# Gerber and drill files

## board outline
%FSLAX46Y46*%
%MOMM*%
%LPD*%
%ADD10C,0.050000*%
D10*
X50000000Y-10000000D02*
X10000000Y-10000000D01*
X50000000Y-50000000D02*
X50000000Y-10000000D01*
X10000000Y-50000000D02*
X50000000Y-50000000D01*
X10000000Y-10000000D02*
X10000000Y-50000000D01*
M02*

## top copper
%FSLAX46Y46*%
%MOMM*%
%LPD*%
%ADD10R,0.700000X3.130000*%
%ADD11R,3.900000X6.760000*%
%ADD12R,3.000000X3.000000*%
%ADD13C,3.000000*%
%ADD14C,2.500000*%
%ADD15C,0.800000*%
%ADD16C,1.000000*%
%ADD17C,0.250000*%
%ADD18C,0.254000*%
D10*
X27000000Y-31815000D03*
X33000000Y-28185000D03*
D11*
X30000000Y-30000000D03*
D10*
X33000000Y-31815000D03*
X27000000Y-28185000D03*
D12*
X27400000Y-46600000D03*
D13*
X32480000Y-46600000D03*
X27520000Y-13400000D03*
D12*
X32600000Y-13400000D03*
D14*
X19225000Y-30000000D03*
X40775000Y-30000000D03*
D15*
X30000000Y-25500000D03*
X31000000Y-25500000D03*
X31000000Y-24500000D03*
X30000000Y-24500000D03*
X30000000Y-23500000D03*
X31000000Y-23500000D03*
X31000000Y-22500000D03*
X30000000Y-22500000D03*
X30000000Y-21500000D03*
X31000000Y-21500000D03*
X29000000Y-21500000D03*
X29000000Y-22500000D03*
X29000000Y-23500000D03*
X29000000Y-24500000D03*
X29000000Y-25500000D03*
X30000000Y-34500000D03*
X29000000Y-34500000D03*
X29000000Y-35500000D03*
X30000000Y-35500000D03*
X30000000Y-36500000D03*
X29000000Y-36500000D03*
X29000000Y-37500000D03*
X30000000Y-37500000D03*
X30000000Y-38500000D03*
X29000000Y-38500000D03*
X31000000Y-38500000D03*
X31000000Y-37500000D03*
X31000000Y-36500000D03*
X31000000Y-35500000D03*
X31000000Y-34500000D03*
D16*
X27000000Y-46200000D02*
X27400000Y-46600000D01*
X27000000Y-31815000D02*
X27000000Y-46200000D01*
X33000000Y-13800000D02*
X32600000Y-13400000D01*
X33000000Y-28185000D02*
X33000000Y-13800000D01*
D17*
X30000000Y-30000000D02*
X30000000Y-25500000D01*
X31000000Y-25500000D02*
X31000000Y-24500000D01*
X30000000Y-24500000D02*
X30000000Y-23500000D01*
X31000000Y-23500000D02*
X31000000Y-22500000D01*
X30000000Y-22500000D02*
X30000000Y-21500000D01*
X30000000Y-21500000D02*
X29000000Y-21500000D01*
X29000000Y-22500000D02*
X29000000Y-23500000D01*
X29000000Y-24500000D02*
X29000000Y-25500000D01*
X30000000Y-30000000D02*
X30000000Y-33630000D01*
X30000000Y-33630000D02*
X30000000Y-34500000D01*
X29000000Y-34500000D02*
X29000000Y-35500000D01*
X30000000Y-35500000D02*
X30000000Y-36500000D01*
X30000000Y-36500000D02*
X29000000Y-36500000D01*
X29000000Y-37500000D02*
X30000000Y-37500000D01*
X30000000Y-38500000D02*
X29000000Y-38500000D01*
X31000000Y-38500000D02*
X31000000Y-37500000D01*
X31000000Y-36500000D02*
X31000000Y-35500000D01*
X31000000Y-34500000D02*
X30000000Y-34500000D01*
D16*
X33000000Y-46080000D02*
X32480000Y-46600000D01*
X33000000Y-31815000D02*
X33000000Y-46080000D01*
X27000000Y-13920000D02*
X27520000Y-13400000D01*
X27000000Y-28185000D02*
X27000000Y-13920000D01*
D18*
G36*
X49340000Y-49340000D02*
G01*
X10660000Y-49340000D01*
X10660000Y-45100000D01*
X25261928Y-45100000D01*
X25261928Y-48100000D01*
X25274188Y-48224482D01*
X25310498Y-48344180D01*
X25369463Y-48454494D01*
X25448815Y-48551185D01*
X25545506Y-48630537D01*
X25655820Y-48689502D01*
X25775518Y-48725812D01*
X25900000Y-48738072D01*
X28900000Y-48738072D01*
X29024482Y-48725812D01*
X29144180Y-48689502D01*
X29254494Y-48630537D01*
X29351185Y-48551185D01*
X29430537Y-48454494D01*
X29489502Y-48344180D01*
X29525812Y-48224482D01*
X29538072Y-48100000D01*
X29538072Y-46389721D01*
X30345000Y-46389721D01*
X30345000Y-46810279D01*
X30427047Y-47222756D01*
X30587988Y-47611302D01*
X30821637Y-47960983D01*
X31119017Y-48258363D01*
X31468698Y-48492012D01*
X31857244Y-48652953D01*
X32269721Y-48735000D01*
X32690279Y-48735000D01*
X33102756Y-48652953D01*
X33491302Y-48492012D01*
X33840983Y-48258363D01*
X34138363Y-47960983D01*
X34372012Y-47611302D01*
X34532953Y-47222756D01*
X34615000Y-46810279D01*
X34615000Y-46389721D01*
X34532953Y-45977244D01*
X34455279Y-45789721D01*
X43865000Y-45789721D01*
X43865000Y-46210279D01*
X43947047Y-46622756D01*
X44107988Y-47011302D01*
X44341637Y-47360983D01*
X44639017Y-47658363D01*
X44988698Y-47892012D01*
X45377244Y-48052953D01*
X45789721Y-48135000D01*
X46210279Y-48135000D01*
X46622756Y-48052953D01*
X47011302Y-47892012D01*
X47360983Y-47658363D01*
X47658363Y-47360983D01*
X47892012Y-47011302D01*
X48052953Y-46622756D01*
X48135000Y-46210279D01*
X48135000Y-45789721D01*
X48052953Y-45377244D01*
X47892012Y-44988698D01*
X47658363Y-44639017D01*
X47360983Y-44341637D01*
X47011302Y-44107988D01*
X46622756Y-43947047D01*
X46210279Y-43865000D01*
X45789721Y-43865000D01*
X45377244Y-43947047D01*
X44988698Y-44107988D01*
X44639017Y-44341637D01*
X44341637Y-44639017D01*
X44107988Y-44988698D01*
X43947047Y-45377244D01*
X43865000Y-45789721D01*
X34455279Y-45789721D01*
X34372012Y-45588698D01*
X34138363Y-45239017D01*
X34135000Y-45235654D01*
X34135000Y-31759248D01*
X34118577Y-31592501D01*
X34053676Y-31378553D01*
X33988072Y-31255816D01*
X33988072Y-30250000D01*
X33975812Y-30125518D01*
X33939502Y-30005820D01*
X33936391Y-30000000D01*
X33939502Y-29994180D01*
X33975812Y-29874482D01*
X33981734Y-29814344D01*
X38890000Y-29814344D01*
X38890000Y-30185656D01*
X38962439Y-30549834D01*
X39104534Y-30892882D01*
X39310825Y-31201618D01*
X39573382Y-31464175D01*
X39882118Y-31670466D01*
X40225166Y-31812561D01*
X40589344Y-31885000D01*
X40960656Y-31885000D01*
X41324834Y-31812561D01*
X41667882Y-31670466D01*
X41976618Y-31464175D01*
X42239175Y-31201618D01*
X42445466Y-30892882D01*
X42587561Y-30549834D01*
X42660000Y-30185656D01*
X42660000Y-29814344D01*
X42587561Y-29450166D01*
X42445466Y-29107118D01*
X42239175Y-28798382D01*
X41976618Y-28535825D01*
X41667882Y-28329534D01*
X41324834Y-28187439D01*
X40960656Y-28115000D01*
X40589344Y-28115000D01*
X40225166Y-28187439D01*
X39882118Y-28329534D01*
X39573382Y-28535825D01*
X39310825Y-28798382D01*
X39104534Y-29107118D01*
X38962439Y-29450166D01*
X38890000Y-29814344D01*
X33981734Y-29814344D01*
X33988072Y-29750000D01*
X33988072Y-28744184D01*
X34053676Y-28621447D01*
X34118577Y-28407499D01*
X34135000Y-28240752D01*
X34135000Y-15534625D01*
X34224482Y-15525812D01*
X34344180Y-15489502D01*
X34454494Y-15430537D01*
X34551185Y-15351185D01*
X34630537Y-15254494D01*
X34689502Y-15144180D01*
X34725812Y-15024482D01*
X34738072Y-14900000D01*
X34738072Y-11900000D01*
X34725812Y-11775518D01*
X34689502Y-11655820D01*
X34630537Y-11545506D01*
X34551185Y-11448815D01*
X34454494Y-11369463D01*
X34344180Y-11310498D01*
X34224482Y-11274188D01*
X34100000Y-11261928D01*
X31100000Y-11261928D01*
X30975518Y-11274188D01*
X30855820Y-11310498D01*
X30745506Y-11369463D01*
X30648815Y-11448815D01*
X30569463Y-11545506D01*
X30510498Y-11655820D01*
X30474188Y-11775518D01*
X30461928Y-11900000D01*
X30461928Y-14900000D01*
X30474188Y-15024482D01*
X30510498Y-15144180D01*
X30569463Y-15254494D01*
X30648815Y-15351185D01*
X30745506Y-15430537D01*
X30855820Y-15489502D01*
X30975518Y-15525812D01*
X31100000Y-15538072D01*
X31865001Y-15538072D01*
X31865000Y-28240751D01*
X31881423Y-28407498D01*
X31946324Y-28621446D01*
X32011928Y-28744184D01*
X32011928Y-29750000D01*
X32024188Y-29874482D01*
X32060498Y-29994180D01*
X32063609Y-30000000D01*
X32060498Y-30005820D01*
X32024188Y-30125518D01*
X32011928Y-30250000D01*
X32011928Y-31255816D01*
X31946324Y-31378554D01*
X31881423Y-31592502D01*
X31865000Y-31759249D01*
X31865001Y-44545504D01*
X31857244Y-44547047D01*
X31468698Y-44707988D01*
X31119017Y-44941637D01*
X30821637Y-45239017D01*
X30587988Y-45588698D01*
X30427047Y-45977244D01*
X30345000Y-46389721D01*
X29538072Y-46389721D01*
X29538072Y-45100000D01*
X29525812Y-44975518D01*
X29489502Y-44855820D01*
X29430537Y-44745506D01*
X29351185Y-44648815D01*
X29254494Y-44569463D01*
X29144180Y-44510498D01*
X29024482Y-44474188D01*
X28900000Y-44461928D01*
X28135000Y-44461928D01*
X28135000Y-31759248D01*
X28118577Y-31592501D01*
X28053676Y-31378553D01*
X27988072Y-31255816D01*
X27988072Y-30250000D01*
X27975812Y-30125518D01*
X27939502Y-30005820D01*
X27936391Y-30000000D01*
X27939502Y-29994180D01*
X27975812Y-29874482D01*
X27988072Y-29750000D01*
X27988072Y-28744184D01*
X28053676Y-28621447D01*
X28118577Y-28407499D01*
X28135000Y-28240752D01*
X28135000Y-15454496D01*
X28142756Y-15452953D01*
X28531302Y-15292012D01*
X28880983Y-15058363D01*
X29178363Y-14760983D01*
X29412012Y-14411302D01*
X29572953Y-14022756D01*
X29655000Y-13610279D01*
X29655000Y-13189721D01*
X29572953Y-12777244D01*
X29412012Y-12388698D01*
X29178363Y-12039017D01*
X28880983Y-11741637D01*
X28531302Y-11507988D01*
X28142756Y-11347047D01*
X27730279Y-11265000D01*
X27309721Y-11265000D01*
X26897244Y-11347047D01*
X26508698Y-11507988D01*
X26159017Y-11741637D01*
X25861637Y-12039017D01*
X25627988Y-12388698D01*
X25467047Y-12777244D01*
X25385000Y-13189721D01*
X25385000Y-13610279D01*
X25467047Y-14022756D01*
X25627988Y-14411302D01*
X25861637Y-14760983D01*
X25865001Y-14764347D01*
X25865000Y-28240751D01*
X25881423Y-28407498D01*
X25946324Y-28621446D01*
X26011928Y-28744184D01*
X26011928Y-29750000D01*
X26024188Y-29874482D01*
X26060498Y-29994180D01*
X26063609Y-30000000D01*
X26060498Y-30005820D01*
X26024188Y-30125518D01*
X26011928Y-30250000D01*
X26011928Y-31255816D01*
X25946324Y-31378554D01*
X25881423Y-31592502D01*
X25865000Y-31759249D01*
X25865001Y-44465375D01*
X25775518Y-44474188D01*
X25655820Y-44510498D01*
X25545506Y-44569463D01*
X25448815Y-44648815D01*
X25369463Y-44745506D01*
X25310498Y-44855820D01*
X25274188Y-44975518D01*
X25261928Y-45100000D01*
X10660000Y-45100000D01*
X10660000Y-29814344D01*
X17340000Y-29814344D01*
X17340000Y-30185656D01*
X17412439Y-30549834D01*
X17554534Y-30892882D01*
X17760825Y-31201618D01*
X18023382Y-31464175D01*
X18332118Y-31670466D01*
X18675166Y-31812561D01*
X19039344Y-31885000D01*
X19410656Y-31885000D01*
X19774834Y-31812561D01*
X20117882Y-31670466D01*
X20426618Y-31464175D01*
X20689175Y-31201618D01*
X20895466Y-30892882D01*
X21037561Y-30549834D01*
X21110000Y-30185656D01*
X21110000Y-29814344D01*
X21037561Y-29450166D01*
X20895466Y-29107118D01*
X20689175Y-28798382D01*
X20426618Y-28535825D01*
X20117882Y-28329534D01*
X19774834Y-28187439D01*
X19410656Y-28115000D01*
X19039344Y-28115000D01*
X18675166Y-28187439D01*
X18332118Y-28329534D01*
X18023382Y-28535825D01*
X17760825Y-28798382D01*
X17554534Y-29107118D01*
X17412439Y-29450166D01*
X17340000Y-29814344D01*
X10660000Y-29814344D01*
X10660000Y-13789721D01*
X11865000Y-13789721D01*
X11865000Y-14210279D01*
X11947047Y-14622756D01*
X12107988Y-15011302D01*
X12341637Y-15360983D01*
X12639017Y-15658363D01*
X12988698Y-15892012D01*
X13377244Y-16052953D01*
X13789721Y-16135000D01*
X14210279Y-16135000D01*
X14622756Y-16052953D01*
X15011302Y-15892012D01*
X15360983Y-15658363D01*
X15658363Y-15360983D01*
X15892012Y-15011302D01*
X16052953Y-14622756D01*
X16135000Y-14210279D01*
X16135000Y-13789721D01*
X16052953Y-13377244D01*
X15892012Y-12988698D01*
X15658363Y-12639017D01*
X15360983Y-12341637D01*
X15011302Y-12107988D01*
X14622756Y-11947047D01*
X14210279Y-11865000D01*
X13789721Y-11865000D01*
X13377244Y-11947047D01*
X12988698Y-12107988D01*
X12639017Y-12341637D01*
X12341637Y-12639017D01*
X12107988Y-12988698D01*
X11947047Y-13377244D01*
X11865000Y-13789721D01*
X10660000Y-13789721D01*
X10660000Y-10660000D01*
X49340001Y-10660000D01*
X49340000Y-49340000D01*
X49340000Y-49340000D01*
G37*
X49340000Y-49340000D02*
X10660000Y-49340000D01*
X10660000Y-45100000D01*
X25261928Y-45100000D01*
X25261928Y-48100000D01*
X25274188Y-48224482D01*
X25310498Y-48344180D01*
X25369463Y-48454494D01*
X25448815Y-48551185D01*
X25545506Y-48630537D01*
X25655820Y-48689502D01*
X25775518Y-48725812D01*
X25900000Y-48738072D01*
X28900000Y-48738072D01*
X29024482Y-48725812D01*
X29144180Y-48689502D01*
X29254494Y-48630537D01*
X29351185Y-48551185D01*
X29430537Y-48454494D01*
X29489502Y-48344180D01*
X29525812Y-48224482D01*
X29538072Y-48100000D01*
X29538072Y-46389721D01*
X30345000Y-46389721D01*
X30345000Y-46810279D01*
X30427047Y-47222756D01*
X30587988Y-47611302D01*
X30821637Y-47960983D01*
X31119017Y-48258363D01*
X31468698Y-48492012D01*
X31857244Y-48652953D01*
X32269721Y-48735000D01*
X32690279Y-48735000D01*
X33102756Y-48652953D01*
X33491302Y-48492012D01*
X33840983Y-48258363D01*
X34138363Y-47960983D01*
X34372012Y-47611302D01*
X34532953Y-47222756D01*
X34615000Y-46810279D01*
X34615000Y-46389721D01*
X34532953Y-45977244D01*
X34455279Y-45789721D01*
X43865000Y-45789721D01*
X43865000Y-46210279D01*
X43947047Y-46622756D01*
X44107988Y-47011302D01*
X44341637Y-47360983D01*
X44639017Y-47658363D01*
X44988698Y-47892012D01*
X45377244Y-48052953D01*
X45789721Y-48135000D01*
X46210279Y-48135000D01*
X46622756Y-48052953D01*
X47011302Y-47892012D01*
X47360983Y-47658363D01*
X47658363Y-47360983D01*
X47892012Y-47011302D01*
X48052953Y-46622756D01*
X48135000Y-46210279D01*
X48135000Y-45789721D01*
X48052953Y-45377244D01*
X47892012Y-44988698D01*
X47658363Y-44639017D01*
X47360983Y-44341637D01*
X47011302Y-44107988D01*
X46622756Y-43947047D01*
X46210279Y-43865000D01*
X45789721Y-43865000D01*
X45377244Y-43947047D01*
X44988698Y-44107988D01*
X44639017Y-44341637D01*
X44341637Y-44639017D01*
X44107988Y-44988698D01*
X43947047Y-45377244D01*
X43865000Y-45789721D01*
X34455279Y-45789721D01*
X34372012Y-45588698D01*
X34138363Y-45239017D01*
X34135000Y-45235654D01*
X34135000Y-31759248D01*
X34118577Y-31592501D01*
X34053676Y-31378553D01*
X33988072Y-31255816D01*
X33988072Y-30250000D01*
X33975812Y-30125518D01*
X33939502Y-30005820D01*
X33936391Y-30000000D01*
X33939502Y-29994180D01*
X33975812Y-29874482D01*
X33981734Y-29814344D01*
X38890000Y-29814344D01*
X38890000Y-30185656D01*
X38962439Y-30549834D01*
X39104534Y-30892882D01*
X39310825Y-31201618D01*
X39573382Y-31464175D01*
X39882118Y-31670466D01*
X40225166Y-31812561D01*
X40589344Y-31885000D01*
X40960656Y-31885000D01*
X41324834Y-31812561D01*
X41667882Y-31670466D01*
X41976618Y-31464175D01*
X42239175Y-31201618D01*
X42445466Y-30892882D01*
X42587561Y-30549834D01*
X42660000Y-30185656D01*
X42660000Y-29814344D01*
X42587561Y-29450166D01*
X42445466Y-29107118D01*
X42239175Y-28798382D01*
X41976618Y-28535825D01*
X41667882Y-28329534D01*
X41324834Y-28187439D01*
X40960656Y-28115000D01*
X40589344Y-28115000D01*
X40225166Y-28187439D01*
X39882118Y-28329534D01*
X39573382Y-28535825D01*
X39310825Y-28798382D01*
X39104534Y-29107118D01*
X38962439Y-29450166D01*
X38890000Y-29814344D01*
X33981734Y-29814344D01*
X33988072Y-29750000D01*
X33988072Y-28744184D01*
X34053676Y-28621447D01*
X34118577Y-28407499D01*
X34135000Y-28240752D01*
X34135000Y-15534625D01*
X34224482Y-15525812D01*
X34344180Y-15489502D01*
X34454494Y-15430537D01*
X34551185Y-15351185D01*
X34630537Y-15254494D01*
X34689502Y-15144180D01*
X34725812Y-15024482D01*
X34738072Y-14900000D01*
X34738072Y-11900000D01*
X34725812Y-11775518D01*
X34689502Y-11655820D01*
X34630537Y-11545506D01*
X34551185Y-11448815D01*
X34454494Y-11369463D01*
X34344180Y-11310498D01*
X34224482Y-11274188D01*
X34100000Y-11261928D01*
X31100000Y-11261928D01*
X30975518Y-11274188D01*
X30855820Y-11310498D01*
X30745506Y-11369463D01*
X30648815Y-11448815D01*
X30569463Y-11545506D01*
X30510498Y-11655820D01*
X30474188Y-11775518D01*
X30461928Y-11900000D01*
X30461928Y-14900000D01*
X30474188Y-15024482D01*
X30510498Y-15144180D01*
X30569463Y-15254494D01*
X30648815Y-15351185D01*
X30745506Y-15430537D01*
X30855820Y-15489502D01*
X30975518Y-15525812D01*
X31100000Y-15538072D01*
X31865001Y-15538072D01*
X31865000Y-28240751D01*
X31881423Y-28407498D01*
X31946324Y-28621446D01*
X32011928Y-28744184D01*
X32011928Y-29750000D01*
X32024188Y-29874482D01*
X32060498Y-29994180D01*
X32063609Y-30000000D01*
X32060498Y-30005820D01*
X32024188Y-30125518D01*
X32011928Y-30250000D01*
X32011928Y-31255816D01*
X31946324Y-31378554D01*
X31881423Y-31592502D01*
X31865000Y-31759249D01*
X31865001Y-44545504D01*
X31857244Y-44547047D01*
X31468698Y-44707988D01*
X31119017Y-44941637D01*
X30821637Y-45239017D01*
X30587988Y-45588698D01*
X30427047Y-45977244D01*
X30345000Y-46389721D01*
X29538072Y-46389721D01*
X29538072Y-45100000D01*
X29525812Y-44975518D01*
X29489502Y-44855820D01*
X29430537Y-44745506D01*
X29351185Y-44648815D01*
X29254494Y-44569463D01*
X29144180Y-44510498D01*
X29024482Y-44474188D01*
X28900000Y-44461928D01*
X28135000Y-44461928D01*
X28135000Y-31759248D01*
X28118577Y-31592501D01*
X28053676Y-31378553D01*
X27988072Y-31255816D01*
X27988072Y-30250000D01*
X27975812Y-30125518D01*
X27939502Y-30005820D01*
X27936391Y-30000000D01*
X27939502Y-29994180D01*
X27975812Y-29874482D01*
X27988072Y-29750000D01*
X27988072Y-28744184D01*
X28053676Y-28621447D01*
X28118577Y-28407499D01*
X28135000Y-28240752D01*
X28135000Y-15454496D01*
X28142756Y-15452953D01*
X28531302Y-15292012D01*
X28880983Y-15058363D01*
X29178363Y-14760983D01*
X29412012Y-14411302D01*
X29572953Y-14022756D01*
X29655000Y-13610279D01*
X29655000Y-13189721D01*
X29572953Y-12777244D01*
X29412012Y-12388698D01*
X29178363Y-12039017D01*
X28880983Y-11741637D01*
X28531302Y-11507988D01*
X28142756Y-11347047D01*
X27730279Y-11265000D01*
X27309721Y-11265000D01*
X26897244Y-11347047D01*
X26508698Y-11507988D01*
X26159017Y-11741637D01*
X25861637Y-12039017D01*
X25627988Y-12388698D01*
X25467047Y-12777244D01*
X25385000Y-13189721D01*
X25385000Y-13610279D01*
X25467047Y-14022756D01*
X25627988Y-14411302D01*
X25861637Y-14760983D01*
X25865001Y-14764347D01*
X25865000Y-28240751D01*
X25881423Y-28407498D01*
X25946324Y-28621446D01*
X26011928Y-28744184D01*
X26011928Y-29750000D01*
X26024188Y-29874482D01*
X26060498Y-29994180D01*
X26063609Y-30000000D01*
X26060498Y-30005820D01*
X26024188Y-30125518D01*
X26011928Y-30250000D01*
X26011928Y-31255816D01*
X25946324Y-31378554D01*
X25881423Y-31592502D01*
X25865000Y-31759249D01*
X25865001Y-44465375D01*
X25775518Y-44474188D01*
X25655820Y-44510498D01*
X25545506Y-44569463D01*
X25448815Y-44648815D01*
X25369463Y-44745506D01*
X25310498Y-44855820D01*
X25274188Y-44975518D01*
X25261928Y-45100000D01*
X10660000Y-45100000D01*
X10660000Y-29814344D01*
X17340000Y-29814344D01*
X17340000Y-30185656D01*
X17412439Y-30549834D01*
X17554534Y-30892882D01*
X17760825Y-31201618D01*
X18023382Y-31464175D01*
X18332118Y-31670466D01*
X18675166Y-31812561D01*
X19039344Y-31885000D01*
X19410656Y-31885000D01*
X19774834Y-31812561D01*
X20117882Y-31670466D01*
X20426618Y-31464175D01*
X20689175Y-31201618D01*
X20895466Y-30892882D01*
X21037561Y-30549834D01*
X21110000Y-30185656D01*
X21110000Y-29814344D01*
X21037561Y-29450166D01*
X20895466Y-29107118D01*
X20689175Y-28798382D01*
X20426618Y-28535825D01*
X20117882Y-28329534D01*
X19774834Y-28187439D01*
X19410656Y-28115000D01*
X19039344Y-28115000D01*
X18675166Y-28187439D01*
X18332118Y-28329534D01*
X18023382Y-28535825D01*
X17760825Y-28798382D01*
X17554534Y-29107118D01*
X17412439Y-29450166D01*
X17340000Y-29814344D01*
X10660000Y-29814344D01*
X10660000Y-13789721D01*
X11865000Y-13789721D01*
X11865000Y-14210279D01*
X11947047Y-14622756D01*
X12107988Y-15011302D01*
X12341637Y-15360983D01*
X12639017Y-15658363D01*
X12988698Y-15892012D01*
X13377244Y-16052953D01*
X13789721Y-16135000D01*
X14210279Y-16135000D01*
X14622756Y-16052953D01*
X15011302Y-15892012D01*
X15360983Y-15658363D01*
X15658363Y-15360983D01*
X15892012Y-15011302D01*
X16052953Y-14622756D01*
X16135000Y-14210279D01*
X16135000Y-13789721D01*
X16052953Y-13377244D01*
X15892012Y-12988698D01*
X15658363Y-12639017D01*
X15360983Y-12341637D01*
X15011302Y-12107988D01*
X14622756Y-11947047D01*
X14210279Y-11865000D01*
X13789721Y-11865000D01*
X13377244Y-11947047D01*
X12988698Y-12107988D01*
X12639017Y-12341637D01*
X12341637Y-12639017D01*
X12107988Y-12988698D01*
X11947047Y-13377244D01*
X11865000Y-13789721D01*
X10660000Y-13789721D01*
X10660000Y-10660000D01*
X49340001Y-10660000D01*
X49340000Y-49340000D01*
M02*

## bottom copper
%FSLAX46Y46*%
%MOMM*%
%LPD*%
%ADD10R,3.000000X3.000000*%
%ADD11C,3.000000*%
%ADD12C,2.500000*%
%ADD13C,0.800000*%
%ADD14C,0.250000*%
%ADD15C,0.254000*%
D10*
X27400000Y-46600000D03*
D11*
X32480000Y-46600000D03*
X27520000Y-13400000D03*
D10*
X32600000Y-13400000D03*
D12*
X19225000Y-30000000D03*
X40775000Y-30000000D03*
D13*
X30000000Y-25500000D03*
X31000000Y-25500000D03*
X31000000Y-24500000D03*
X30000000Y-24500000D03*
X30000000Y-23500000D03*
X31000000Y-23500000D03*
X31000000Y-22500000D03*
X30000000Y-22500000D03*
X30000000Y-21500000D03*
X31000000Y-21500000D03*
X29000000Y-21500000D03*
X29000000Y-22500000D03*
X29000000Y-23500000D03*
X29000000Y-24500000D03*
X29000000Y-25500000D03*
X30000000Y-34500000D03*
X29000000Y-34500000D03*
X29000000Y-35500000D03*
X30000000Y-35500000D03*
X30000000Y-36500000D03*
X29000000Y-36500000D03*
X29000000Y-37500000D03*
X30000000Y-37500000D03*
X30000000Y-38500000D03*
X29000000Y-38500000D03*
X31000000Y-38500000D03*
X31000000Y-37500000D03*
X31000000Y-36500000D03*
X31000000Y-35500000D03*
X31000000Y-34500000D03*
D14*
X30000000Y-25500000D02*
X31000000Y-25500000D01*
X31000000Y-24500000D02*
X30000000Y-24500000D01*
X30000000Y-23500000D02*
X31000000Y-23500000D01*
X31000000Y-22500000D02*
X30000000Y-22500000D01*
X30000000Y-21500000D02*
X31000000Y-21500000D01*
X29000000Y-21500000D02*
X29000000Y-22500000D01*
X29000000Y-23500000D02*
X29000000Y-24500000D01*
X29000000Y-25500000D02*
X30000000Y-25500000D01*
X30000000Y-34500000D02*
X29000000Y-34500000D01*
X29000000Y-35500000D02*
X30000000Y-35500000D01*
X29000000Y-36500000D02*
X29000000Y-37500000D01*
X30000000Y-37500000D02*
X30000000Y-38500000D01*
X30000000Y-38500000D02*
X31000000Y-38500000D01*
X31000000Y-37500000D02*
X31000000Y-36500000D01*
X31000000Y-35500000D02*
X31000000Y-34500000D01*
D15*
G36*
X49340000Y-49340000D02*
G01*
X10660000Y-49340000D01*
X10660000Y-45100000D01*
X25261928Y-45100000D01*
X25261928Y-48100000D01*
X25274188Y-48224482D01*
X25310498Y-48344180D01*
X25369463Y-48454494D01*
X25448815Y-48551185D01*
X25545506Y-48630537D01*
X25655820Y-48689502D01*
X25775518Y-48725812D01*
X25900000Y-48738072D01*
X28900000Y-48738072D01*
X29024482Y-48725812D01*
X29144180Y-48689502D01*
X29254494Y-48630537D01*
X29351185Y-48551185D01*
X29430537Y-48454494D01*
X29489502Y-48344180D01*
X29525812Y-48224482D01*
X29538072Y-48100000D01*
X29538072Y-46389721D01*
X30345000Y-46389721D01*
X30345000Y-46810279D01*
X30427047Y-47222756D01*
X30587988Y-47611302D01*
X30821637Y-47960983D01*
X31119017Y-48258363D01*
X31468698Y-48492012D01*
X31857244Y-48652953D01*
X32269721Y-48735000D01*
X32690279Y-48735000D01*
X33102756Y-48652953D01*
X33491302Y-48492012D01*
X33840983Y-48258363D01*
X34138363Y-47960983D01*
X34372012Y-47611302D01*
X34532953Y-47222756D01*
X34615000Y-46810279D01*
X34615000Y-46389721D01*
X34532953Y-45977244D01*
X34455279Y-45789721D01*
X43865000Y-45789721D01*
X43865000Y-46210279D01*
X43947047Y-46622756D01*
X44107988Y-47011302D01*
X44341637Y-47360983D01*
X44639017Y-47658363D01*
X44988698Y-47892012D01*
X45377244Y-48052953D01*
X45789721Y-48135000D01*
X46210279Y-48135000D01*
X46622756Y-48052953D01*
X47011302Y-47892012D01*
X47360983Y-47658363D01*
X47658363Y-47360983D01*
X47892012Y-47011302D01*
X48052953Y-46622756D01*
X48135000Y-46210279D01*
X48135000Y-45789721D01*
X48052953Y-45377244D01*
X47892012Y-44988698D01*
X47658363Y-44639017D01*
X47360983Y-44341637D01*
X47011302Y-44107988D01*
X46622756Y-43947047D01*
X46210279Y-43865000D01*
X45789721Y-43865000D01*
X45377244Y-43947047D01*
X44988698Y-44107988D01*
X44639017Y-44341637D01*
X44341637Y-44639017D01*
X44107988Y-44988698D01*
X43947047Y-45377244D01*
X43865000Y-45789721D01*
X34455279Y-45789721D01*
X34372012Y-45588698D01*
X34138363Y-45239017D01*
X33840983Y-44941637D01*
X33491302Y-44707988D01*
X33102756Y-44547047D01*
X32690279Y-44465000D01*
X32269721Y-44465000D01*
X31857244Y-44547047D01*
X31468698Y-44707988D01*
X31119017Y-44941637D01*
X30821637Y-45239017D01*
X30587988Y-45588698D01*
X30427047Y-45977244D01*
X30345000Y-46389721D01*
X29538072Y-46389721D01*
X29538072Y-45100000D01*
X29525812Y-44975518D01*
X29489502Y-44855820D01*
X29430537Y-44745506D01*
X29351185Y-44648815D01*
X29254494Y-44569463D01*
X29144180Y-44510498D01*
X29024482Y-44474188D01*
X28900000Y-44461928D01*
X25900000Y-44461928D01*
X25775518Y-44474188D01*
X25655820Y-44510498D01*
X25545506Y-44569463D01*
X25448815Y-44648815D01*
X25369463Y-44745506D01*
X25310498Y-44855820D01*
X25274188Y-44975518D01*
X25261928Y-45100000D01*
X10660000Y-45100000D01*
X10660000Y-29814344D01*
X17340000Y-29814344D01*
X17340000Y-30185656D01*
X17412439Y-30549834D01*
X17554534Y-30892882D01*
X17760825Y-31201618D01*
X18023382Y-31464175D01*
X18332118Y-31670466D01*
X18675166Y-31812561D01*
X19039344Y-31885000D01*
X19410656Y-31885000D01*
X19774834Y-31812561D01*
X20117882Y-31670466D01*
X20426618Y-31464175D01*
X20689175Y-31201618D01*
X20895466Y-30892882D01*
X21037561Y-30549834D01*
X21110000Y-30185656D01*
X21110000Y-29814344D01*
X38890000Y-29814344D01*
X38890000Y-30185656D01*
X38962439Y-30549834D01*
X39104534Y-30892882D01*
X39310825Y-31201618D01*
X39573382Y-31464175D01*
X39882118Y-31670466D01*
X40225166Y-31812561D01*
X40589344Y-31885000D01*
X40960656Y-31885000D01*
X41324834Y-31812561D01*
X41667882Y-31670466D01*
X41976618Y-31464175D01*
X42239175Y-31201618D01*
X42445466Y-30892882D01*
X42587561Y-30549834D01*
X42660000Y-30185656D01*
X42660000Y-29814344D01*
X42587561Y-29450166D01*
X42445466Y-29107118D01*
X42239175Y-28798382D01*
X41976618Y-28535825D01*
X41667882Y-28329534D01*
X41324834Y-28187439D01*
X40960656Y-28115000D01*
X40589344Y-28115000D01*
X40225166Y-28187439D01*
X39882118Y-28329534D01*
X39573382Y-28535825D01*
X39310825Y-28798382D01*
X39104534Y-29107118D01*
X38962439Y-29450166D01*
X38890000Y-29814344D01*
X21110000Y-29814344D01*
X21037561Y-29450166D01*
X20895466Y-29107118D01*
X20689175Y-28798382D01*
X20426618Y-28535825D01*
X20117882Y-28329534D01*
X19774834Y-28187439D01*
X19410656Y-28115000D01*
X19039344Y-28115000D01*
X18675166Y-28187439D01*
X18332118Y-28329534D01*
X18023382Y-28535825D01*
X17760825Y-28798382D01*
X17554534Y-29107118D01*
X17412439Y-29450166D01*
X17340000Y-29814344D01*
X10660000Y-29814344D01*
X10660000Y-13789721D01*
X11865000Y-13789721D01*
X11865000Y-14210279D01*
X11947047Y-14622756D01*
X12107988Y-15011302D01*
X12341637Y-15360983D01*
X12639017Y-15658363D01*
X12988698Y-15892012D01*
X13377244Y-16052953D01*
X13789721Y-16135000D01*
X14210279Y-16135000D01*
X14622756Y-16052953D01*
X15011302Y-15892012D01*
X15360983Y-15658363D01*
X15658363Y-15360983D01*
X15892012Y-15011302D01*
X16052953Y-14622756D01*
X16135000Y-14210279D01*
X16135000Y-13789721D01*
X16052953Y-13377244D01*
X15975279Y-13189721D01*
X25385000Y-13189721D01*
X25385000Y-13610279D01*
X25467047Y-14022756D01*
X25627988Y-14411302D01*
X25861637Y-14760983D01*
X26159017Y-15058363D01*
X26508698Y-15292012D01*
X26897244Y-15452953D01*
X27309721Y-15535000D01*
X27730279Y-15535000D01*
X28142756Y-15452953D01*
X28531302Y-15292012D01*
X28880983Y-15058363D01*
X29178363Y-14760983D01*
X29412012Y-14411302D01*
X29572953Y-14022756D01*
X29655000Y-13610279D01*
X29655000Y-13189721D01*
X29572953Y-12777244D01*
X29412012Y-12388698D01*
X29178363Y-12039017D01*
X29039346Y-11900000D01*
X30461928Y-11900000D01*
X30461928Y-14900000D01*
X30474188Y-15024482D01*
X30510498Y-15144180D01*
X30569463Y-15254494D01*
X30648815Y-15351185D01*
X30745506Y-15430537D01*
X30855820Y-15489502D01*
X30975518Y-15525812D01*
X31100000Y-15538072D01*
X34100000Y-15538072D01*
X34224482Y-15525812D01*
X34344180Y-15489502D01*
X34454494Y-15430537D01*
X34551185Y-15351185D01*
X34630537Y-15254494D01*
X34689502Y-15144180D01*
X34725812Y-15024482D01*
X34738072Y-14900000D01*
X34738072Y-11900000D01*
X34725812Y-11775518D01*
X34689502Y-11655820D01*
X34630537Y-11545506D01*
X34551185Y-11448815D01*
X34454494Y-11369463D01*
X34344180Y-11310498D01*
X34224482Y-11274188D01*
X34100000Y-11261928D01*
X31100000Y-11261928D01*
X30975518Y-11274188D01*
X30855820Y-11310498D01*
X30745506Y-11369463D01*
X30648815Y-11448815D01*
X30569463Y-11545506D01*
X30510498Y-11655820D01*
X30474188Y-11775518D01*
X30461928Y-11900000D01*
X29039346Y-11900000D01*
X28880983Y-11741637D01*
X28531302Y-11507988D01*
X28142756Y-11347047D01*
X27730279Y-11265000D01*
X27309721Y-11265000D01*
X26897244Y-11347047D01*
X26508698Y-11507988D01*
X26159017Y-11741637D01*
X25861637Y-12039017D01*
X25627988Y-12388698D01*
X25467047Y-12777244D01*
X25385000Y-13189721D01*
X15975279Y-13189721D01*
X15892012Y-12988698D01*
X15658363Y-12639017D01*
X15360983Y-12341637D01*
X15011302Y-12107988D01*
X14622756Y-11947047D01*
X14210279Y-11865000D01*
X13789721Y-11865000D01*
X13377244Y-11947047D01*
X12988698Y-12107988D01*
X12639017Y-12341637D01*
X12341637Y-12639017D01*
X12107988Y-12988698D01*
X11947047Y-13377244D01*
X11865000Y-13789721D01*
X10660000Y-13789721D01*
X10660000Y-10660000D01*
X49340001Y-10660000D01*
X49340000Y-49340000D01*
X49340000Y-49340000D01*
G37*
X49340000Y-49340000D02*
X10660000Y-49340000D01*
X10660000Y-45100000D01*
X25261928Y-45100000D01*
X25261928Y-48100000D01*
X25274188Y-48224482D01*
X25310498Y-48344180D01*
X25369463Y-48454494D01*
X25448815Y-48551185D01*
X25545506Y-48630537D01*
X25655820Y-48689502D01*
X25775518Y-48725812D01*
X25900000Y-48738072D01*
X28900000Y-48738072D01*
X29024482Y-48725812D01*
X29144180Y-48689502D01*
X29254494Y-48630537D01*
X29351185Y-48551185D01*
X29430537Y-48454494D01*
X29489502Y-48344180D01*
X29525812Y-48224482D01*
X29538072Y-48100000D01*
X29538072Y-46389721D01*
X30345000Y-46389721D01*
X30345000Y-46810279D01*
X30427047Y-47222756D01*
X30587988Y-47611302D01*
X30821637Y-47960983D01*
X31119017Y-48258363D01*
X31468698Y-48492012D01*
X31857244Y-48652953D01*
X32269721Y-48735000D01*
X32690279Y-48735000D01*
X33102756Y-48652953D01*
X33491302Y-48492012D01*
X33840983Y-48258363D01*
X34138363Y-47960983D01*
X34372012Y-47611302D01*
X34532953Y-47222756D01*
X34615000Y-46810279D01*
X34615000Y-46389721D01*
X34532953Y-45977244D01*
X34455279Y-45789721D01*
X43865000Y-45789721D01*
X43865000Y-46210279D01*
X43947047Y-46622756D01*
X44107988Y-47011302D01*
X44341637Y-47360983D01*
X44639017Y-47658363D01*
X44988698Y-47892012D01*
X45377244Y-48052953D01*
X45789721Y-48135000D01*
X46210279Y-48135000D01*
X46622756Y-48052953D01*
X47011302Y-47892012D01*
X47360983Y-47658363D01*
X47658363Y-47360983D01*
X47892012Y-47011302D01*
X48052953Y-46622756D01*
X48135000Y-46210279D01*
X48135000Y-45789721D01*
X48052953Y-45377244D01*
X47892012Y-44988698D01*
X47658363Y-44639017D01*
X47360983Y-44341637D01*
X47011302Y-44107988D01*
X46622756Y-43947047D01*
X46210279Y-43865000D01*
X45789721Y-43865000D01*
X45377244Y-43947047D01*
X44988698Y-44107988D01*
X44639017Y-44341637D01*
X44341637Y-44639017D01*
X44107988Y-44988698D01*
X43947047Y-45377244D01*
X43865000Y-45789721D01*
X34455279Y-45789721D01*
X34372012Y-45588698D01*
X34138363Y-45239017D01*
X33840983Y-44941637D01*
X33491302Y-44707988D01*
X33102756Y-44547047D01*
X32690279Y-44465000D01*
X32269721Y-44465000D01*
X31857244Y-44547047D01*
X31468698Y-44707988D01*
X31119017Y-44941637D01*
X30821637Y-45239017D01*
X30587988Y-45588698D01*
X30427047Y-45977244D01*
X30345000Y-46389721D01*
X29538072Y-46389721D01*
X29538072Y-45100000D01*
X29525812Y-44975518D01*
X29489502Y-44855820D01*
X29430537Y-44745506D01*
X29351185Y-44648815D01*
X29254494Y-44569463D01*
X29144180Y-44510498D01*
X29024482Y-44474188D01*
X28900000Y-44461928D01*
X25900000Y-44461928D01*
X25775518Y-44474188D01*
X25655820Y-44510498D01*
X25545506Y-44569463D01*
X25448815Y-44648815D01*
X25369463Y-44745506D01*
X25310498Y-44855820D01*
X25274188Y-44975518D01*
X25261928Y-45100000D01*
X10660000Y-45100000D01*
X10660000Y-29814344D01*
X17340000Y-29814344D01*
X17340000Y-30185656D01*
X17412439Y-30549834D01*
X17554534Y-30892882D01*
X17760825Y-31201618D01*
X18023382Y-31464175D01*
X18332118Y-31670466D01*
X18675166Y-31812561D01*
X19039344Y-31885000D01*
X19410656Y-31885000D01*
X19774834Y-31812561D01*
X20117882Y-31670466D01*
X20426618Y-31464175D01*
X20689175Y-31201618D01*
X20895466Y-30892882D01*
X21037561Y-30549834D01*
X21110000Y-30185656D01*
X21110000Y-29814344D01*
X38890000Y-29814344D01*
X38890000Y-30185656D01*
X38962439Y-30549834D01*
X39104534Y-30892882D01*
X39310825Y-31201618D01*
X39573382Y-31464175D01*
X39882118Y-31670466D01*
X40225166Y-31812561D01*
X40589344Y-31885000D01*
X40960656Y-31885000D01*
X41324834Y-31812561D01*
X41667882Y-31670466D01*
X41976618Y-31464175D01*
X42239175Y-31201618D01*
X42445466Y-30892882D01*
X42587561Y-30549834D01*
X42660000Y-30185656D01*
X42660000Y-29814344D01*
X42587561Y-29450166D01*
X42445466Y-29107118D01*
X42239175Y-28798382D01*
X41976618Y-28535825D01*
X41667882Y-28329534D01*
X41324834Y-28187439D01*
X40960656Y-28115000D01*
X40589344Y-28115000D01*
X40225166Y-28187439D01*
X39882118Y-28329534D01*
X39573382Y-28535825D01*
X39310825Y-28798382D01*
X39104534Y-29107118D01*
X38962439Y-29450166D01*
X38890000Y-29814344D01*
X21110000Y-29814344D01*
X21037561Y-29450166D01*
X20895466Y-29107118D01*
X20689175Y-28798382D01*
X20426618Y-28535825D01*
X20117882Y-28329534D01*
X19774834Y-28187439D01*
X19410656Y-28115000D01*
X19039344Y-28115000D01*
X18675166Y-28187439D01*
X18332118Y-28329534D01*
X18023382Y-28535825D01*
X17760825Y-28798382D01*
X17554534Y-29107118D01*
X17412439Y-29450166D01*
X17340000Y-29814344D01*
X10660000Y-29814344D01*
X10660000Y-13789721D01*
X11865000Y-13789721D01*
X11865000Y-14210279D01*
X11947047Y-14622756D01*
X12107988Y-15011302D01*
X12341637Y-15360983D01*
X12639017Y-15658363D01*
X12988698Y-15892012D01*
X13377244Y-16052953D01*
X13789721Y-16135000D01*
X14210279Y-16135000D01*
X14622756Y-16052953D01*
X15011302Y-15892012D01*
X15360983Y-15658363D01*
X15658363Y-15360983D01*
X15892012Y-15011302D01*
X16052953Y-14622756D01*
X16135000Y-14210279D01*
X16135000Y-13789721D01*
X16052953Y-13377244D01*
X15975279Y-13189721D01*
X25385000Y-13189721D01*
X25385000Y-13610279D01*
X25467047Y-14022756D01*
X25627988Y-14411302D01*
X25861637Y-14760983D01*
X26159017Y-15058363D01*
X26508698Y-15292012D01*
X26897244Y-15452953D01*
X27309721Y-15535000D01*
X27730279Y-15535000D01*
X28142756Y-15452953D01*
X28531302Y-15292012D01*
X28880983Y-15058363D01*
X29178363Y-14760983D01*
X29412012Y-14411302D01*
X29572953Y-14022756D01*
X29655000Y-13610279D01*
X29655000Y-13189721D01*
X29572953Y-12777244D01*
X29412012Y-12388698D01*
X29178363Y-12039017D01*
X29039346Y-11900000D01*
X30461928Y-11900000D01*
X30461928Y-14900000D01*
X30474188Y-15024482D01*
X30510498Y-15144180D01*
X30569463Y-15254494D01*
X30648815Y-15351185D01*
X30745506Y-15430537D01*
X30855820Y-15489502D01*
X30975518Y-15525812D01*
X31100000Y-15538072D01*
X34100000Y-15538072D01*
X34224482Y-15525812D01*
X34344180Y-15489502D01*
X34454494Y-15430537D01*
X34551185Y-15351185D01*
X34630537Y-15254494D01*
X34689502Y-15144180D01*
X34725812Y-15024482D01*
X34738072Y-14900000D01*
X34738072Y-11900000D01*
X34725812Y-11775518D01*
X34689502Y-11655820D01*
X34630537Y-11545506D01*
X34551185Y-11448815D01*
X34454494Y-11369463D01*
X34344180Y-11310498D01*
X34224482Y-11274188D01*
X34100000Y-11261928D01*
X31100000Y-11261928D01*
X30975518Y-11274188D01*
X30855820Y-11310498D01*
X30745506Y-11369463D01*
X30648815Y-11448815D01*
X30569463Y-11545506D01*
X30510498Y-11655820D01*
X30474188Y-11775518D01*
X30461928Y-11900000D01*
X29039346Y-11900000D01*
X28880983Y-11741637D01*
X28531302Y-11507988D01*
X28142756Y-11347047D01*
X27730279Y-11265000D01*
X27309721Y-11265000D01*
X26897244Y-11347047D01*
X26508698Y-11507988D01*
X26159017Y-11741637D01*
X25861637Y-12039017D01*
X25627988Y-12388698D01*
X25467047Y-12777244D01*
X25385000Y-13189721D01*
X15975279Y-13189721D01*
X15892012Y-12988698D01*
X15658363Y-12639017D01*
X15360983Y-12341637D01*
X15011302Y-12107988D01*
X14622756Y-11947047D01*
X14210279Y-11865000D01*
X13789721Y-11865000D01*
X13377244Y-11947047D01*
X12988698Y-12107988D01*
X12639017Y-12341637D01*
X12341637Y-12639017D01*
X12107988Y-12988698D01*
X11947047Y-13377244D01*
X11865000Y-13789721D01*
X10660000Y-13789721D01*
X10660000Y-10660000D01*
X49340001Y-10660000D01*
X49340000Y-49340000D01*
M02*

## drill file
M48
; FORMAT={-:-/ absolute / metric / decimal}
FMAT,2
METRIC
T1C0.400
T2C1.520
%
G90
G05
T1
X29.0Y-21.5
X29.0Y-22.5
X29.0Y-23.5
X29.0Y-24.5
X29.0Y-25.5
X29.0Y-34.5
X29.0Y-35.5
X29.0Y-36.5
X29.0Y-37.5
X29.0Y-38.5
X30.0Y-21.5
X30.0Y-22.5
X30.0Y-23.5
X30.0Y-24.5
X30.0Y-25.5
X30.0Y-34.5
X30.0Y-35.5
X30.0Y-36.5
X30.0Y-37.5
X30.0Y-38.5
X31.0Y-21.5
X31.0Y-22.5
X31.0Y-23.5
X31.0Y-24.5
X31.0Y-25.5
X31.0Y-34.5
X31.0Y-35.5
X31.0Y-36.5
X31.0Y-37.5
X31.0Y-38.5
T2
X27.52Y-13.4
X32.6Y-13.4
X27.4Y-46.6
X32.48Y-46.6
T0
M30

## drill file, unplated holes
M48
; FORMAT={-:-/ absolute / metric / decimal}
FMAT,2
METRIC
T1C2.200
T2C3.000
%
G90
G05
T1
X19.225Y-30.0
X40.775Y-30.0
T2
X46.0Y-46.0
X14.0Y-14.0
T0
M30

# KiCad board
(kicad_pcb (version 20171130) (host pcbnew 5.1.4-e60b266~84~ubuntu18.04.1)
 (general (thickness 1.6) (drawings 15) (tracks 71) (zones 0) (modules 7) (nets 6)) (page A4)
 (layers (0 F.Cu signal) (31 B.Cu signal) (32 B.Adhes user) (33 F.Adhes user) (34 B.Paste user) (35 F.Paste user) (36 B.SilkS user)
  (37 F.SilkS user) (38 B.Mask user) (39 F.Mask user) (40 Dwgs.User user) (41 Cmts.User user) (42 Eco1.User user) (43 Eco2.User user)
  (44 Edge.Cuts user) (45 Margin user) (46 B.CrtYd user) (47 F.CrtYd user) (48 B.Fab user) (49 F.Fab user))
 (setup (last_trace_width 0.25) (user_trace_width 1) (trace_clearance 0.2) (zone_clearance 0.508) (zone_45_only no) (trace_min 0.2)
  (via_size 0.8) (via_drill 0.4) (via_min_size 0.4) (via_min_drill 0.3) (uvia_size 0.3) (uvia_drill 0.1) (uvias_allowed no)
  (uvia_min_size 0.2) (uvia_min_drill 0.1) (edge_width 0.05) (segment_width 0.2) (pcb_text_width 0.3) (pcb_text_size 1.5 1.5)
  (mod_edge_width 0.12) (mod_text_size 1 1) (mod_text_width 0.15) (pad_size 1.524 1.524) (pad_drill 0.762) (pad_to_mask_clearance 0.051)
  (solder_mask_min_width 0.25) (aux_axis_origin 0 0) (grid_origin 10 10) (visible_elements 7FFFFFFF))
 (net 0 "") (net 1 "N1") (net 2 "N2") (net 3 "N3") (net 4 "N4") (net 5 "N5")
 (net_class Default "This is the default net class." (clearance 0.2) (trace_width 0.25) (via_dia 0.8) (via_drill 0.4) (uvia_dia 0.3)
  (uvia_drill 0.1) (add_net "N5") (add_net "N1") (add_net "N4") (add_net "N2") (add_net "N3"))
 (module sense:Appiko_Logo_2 (layer F.Cu) (at 14.6 32.9 90)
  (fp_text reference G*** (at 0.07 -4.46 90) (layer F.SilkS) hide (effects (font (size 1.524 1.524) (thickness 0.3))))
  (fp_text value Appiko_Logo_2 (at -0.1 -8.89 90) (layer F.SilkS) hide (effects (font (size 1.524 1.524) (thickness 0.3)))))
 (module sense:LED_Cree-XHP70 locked (layer F.Cu) (at 30 30)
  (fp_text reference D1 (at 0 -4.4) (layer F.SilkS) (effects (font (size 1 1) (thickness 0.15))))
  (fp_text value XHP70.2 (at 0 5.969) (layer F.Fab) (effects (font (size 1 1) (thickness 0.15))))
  (pad 2 smd rect (at -3 1.815) (size 0.7 3.13) (layers F.Cu F.Paste F.Mask) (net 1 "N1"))
  (pad 4 smd rect (at 3 -1.815) (size 0.7 3.13) (layers F.Cu F.Paste F.Mask) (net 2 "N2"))
  (pad 5 smd rect (at 0 0) (size 3.9 6.76) (layers F.Cu F.Mask) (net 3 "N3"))
  (pad 3 smd rect (at 3 1.815) (size 0.7 3.13) (layers F.Cu B.Paste F.Mask) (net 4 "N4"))
  (pad 1 smd rect (at -3 -1.815) (size 0.7 3.13) (layers F.Cu F.Paste F.Mask) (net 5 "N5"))
  (pad 3 smd rect (at -0.77 -2.31) (size 1.29 1.29) (layers F.Paste) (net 4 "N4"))
  (pad 3 smd rect (at 0.77 -2.31) (size 1.29 1.29) (layers F.Paste) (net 4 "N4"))
  (pad 3 smd rect (at -0.77 -0.77) (size 1.29 1.29) (layers F.Paste) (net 4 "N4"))
  (pad 3 smd rect (at 0.77 -0.77) (size 1.29 1.29) (layers F.Paste) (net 4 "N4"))
  (pad 3 smd rect (at -0.77 0.77) (size 1.29 1.29) (layers F.Paste) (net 4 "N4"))
  (pad 3 smd rect (at 0.77 0.77) (size 1.29 1.29) (layers F.Paste) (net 4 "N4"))
  (pad 3 smd rect (at -0.77 2.31) (size 1.29 1.29) (layers F.Paste) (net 4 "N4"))
  (pad 3 smd rect (at 0.77 2.31) (size 1.29 1.29) (layers F.Paste) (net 4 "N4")))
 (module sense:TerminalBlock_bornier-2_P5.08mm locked (layer F.Cu) (at 27.4 46.6)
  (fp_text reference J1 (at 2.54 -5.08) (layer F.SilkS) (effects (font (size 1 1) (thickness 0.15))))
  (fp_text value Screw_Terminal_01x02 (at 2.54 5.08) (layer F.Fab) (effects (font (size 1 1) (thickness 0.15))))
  (pad 1 thru_hole rect (at 0 0) (size 3 3) (drill 1.52) (layers *.Cu *.Mask) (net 1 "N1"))
  (pad 2 thru_hole circle (at 5.08 0) (size 3 3) (drill 1.52) (layers *.Cu *.Mask) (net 4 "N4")))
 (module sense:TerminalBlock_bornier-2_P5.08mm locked (layer F.Cu) (at 32.6 13.4 180)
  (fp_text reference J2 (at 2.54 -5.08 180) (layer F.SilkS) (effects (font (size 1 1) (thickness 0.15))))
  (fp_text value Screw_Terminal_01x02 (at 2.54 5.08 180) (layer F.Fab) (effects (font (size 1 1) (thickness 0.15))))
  (pad 2 thru_hole circle (at 5.08 0 180) (size 3 3) (drill 1.52) (layers *.Cu *.Mask) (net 5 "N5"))
  (pad 1 thru_hole rect (at 0 0 180) (size 3 3) (drill 1.52) (layers *.Cu *.Mask) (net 2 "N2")))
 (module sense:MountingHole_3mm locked (layer F.Cu) (at 14 14)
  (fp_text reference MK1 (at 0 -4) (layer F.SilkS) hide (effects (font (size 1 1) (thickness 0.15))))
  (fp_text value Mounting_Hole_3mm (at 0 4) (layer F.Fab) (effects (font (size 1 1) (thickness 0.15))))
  (pad 1 np_thru_hole circle (at 0 0) (size 3 3) (drill 3) (layers *.Cu *.Mask)))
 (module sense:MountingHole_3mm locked (layer F.Cu) (at 46 46)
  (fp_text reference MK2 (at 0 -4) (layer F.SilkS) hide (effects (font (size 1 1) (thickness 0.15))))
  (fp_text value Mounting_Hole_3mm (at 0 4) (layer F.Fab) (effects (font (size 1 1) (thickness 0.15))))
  (pad 1 np_thru_hole circle (at 0 0) (size 3 3) (drill 3) (layers *.Cu *.Mask)))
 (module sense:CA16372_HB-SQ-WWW (layer F.Cu) (at 30 30)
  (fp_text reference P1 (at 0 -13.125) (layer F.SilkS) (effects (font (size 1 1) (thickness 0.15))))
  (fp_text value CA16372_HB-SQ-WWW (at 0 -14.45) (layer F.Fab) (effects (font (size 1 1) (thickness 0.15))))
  (pad "" np_thru_hole circle (at -10.775 0) (size 2.5 2.5) (drill 2.2) (layers *.Cu *.Mask))
  (pad "" np_thru_hole circle (at 10.775 0) (size 2.5 2.5) (drill 2.2) (layers *.Cu *.Mask)))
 (gr_line (start 50 10) (end 10 10) (layer Edge.Cuts) (width 0.05))
 (gr_line (start 50 50) (end 50 10) (layer Edge.Cuts) (width 0.05))
 (gr_line (start 10 50) (end 50 50) (layer Edge.Cuts) (width 0.05))
 (gr_line (start 10 10) (end 10 50) (layer Edge.Cuts) (width 0.05))
 (segment (start 27 46.2) (end 27.4 46.6) (width 1) (layer F.Cu) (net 1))
 (segment (start 27 31.815) (end 27 46.2) (width 1) (layer F.Cu) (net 1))
 (segment (start 33 13.8) (end 32.6 13.4) (width 1) (layer F.Cu) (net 2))
 (segment (start 33 28.185) (end 33 13.8) (width 1) (layer F.Cu) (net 2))
 (via (at 30 25.5) (size 0.8) (drill 0.4) (layers F.Cu B.Cu) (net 3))
 (segment (start 30 30) (end 30 25.5) (width 0.25) (layer F.Cu) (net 3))
 (via (at 31 25.5) (size 0.8) (drill 0.4) (layers F.Cu B.Cu) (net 3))
 (segment (start 30 25.5) (end 31 25.5) (width 0.25) (layer B.Cu) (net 3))
 (via (at 31 24.5) (size 0.8) (drill 0.4) (layers F.Cu B.Cu) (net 3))
 (segment (start 31 25.5) (end 31 24.5) (width 0.25) (layer F.Cu) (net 3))
 (via (at 30 24.5) (size 0.8) (drill 0.4) (layers F.Cu B.Cu) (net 3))
 (segment (start 31 24.5) (end 30 24.5) (width 0.25) (layer B.Cu) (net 3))
 (via (at 30 23.5) (size 0.8) (drill 0.4) (layers F.Cu B.Cu) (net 3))
 (segment (start 30 24.5) (end 30 23.5) (width 0.25) (layer F.Cu) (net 3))
 (via (at 31 23.5) (size 0.8) (drill 0.4) (layers F.Cu B.Cu) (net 3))
 (segment (start 30 23.5) (end 31 23.5) (width 0.25) (layer B.Cu) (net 3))
 (via (at 31 22.5) (size 0.8) (drill 0.4) (layers F.Cu B.Cu) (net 3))
 (segment (start 31 23.5) (end 31 22.5) (width 0.25) (layer F.Cu) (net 3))
 (via (at 30 22.5) (size 0.8) (drill 0.4) (layers F.Cu B.Cu) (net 3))
 (segment (start 31 22.5) (end 30 22.5) (width 0.25) (layer B.Cu) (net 3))
 (via (at 30 21.5) (size 0.8) (drill 0.4) (layers F.Cu B.Cu) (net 3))
 (segment (start 30 22.5) (end 30 21.5) (width 0.25) (layer F.Cu) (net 3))
 (via (at 31 21.5) (size 0.8) (drill 0.4) (layers F.Cu B.Cu) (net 3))
 (segment (start 30 21.5) (end 31 21.5) (width 0.25) (layer B.Cu) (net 3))
 (via (at 29 21.5) (size 0.8) (drill 0.4) (layers F.Cu B.Cu) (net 3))
 (segment (start 30 21.5) (end 29 21.5) (width 0.25) (layer F.Cu) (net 3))
 (via (at 29 22.5) (size 0.8) (drill 0.4) (layers F.Cu B.Cu) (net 3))
 (segment (start 29 21.5) (end 29 22.5) (width 0.25) (layer B.Cu) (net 3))
 (via (at 29 23.5) (size 0.8) (drill 0.4) (layers F.Cu B.Cu) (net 3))
 (segment (start 29 22.5) (end 29 23.5) (width 0.25) (layer F.Cu) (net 3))
 (via (at 29 24.5) (size 0.8) (drill 0.4) (layers F.Cu B.Cu) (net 3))
 (segment (start 29 23.5) (end 29 24.5) (width 0.25) (layer B.Cu) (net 3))
 (via (at 29 25.5) (size 0.8) (drill 0.4) (layers F.Cu B.Cu) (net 3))
 (segment (start 29 24.5) (end 29 25.5) (width 0.25) (layer F.Cu) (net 3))
 (segment (start 29 25.5) (end 30 25.5) (width 0.25) (layer B.Cu) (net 3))
 (via (at 30 34.5) (size 0.8) (drill 0.4) (layers F.Cu B.Cu) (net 3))
 (segment (start 30 30) (end 30 33.63) (width 0.25) (layer F.Cu) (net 3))
 (segment (start 30 33.63) (end 30 34.5) (width 0.25) (layer F.Cu) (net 3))
 (via (at 29 34.5) (size 0.8) (drill 0.4) (layers F.Cu B.Cu) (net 3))
 (segment (start 30 34.5) (end 29 34.5) (width 0.25) (layer B.Cu) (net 3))
 (via (at 29 35.5) (size 0.8) (drill 0.4) (layers F.Cu B.Cu) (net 3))
 (segment (start 29 34.5) (end 29 35.5) (width 0.25) (layer F.Cu) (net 3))
 (via (at 30 35.5) (size 0.8) (drill 0.4) (layers F.Cu B.Cu) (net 3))
 (segment (start 29 35.5) (end 30 35.5) (width 0.25) (layer B.Cu) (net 3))
 (via (at 30 36.5) (size 0.8) (drill 0.4) (layers F.Cu B.Cu) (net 3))
 (segment (start 30 35.5) (end 30 36.5) (width 0.25) (layer F.Cu) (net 3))
 (via (at 29 36.5) (size 0.8) (drill 0.4) (layers F.Cu B.Cu) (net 3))
 (segment (start 30 36.5) (end 29 36.5) (width 0.25) (layer F.Cu) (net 3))
 (via (at 29 37.5) (size 0.8) (drill 0.4) (layers F.Cu B.Cu) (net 3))
 (segment (start 29 36.5) (end 29 37.5) (width 0.25) (layer B.Cu) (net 3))
 (via (at 30 37.5) (size 0.8) (drill 0.4) (layers F.Cu B.Cu) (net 3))
 (segment (start 29 37.5) (end 30 37.5) (width 0.25) (layer F.Cu) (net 3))
 (via (at 30 38.5) (size 0.8) (drill 0.4) (layers F.Cu B.Cu) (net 3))
 (segment (start 30 37.5) (end 30 38.5) (width 0.25) (layer B.Cu) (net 3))
 (via (at 29 38.5) (size 0.8) (drill 0.4) (layers F.Cu B.Cu) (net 3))
 (segment (start 30 38.5) (end 29 38.5) (width 0.25) (layer F.Cu) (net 3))
 (via (at 31 38.5) (size 0.8) (drill 0.4) (layers F.Cu B.Cu) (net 3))
 (segment (start 30 38.5) (end 31 38.5) (width 0.25) (layer B.Cu) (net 3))
 (via (at 31 37.5) (size 0.8) (drill 0.4) (layers F.Cu B.Cu) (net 3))
 (segment (start 31 38.5) (end 31 37.5) (width 0.25) (layer F.Cu) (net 3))
 (via (at 31 36.5) (size 0.8) (drill 0.4) (layers F.Cu B.Cu) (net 3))
 (segment (start 31 37.5) (end 31 36.5) (width 0.25) (layer B.Cu) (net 3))
 (via (at 31 35.5) (size 0.8) (drill 0.4) (layers F.Cu B.Cu) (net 3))
 (segment (start 31 36.5) (end 31 35.5) (width 0.25) (layer F.Cu) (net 3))
 (via (at 31 34.5) (size 0.8) (drill 0.4) (layers F.Cu B.Cu) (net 3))
 (segment (start 31 35.5) (end 31 34.5) (width 0.25) (layer B.Cu) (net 3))
 (segment (start 31 34.5) (end 30 34.5) (width 0.25) (layer F.Cu) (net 3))
 (segment (start 33 46.08) (end 32.48 46.6) (width 1) (layer F.Cu) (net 4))
 (segment (start 33 31.815) (end 33 46.08) (width 1) (layer F.Cu) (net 4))
 (segment (start 27 13.92) (end 27.52 13.4) (width 1) (layer F.Cu) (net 5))
 (segment (start 27 28.185) (end 27 13.92) (width 1) (layer F.Cu) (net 5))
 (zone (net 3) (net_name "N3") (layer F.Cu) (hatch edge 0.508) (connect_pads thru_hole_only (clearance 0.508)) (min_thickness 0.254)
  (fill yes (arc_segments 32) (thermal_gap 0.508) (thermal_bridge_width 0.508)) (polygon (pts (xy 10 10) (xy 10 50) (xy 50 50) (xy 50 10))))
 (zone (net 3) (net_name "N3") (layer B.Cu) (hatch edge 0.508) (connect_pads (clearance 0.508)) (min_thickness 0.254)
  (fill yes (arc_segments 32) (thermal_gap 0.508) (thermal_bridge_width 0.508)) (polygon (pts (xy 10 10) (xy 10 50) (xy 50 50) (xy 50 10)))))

